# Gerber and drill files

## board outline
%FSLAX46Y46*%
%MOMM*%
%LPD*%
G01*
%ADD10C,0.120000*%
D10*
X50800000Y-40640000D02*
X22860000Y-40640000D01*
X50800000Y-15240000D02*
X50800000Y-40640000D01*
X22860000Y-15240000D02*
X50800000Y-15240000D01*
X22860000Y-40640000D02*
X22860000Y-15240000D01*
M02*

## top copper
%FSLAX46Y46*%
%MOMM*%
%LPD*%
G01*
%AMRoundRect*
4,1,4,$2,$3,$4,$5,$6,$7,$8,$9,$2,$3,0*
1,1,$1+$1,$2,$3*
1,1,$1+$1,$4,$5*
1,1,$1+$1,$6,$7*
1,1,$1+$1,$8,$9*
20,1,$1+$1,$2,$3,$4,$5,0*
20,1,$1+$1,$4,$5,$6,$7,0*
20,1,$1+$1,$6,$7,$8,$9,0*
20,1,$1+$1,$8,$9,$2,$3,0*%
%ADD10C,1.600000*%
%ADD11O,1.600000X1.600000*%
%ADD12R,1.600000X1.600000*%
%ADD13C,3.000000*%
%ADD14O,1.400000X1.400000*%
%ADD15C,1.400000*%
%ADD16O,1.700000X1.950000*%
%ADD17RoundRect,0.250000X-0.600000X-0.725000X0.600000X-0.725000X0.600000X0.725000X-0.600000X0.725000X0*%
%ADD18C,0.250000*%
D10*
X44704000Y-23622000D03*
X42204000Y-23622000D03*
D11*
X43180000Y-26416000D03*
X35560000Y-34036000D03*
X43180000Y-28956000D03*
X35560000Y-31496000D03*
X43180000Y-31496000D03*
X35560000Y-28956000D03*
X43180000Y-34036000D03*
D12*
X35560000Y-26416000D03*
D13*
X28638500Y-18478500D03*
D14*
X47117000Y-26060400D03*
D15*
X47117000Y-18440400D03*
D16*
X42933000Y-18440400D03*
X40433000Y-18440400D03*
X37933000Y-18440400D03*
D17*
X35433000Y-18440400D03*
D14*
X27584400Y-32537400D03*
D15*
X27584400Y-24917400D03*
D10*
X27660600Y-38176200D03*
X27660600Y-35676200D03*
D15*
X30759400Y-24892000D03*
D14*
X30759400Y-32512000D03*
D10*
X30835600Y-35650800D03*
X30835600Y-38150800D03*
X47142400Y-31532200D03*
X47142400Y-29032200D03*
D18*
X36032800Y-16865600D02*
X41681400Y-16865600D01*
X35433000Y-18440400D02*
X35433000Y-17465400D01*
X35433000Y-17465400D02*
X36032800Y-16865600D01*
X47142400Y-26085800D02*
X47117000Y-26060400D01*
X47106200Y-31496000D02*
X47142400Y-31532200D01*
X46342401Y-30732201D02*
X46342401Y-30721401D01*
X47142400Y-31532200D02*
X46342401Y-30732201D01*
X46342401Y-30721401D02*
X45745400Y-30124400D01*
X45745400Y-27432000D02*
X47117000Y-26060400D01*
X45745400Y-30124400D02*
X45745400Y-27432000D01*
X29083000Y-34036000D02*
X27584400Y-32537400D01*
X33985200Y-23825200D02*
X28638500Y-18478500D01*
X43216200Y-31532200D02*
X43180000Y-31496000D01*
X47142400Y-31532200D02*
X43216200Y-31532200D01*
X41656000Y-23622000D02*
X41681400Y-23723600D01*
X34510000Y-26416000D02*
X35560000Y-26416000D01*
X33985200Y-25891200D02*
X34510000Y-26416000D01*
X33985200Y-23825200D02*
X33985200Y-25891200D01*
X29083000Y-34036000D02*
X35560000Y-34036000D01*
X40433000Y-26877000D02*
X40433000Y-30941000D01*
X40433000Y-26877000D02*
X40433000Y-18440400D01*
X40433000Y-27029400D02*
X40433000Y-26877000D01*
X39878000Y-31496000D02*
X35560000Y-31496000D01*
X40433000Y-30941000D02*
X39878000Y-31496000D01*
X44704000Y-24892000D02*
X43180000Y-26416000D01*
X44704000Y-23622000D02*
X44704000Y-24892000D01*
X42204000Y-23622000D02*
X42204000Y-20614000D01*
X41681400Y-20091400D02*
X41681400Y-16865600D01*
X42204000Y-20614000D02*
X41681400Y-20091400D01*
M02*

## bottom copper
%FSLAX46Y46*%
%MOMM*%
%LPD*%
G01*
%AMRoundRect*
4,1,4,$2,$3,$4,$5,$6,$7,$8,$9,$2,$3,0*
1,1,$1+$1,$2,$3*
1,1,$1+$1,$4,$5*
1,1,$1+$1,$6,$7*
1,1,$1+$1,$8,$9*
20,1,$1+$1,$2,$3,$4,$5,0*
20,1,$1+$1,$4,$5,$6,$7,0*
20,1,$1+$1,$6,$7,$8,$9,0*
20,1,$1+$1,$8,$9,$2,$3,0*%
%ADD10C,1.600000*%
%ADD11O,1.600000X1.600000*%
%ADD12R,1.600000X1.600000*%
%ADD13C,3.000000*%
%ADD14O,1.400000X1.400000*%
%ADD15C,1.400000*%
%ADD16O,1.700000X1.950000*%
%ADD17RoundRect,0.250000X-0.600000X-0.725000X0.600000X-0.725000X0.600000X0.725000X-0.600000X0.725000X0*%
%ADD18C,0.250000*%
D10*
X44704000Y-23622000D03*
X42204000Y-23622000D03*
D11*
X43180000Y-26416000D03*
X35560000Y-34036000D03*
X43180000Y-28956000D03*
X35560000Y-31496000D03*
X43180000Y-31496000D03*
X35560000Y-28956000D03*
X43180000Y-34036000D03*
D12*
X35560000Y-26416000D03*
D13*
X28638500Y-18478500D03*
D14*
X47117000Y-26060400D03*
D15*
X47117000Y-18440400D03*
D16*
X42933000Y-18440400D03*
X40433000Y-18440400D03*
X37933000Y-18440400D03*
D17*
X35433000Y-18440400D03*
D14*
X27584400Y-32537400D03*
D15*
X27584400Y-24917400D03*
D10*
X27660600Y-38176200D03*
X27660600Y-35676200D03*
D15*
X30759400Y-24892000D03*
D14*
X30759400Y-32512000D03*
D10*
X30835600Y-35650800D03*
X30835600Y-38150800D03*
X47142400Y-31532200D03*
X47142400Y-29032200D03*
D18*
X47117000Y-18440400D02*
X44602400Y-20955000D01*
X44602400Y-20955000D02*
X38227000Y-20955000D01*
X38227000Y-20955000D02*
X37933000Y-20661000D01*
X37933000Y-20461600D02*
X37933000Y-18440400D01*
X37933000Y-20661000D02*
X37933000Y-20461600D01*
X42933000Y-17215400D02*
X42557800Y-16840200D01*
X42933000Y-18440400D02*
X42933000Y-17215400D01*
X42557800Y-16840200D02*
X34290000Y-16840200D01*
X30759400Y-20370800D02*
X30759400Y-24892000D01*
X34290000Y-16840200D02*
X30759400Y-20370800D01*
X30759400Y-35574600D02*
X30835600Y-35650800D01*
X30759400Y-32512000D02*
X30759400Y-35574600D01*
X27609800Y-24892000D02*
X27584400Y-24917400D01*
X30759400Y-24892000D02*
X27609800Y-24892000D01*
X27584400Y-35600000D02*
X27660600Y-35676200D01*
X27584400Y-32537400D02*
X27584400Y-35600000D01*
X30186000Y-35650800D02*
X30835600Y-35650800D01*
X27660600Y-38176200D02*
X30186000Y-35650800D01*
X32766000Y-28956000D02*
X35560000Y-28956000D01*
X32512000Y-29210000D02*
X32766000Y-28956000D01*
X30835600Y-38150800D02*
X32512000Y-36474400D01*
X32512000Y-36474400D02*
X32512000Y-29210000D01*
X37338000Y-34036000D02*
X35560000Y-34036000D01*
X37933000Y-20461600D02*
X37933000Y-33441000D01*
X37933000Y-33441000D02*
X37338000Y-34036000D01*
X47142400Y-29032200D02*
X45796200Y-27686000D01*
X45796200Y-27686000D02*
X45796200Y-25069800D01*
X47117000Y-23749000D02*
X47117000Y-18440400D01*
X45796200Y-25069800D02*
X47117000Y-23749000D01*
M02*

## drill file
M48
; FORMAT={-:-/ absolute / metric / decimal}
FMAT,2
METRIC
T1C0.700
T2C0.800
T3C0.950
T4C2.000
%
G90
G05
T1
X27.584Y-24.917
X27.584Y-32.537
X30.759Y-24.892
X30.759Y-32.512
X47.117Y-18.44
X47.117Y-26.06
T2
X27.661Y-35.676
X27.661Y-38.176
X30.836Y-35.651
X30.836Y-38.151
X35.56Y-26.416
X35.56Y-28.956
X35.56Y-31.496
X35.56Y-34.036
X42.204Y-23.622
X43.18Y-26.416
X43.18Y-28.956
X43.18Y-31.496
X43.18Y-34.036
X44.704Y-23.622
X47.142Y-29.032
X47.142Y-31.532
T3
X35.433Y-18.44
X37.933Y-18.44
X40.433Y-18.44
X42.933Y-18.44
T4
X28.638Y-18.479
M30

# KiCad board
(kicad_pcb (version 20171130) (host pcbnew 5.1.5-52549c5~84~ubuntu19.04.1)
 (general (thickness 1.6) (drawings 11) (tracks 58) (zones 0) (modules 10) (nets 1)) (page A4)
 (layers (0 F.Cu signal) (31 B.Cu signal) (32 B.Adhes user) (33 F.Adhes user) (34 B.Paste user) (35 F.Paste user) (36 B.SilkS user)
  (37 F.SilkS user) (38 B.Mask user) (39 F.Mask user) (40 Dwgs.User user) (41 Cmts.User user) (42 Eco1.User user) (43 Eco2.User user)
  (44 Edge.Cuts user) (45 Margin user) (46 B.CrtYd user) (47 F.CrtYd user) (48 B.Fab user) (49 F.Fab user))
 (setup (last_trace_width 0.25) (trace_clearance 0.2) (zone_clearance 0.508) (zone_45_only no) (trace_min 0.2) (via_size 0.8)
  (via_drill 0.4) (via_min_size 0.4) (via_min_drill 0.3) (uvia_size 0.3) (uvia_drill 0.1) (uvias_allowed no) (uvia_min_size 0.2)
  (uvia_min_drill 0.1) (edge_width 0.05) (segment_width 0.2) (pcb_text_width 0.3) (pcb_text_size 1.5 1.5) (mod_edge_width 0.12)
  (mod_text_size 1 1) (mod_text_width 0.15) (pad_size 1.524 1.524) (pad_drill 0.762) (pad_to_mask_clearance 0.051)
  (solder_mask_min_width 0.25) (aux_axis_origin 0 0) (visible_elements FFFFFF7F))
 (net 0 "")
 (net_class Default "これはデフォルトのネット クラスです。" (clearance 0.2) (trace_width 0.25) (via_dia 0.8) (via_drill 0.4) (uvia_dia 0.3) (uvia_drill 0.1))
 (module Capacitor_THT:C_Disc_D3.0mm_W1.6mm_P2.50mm (layer F.Cu) (at 44.704 23.622 180)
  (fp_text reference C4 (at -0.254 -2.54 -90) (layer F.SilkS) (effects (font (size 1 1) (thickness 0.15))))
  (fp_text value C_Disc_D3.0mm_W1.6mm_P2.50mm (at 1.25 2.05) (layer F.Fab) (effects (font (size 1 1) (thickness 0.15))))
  (pad 1 thru_hole circle (at 0 0 180) (size 1.6 1.6) (drill 0.8) (layers *.Cu *.Mask))
  (pad 2 thru_hole circle (at 2.5 0 180) (size 1.6 1.6) (drill 0.8) (layers *.Cu *.Mask)))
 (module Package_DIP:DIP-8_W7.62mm (layer F.Cu) (at 35.56 26.416)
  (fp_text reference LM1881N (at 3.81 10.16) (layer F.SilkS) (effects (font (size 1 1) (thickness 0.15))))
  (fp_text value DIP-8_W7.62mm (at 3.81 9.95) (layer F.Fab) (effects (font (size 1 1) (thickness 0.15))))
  (pad 8 thru_hole oval (at 7.62 0) (size 1.6 1.6) (drill 0.8) (layers *.Cu *.Mask))
  (pad 4 thru_hole oval (at 0 7.62) (size 1.6 1.6) (drill 0.8) (layers *.Cu *.Mask))
  (pad 7 thru_hole oval (at 7.62 2.54) (size 1.6 1.6) (drill 0.8) (layers *.Cu *.Mask))
  (pad 3 thru_hole oval (at 0 5.08) (size 1.6 1.6) (drill 0.8) (layers *.Cu *.Mask))
  (pad 6 thru_hole oval (at 7.62 5.08) (size 1.6 1.6) (drill 0.8) (layers *.Cu *.Mask))
  (pad 2 thru_hole oval (at 0 2.54) (size 1.6 1.6) (drill 0.8) (layers *.Cu *.Mask))
  (pad 5 thru_hole oval (at 7.62 7.62) (size 1.6 1.6) (drill 0.8) (layers *.Cu *.Mask))
  (pad 1 thru_hole rect (at 0 0) (size 1.6 1.6) (drill 0.8) (layers *.Cu *.Mask)))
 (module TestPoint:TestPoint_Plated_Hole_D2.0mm (layer F.Cu) (at 28.6385 18.4785)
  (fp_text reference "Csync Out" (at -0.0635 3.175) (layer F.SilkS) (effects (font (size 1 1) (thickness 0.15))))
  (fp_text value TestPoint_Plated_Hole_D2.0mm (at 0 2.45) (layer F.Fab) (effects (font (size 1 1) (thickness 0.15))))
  (pad 1 thru_hole circle (at 0 0) (size 3 3) (drill 2) (layers *.Cu *.Mask)))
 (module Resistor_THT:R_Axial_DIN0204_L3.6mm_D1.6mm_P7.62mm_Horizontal (layer F.Cu) (at 47.117 18.4404 270)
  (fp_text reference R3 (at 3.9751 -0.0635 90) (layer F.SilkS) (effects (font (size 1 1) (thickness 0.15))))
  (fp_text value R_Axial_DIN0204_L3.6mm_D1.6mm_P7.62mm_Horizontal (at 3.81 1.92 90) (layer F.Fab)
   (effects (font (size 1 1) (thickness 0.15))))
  (pad 2 thru_hole oval (at 7.62 0 270) (size 1.4 1.4) (drill 0.7) (layers *.Cu *.Mask))
  (pad 1 thru_hole circle (at 0 0 270) (size 1.4 1.4) (drill 0.7) (layers *.Cu *.Mask)))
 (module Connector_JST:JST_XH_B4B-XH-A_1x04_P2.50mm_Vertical (layer F.Cu) (at 35.433 18.4404)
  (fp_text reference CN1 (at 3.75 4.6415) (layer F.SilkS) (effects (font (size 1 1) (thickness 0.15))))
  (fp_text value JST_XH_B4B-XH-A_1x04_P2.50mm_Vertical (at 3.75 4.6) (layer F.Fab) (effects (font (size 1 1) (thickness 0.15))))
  (pad 4 thru_hole oval (at 7.5 0) (size 1.7 1.95) (drill 0.95) (layers *.Cu *.Mask))
  (pad 3 thru_hole oval (at 5 0) (size 1.7 1.95) (drill 0.95) (layers *.Cu *.Mask))
  (pad 2 thru_hole oval (at 2.5 0) (size 1.7 1.95) (drill 0.95) (layers *.Cu *.Mask))
  (pad 1 thru_hole roundrect (at 0 0) (size 1.7 1.95) (drill 0.95) (layers *.Cu *.Mask) (roundrect_rratio 0.147059)))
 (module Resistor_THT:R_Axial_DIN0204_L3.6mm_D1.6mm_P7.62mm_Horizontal (layer F.Cu) (at 27.5844 24.9174 270)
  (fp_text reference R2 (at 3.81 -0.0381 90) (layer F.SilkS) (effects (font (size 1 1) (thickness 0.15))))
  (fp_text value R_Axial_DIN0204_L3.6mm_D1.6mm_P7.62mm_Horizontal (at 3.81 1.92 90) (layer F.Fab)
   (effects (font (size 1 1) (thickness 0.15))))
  (pad 2 thru_hole oval (at 7.62 0 270) (size 1.4 1.4) (drill 0.7) (layers *.Cu *.Mask))
  (pad 1 thru_hole circle (at 0 0 270) (size 1.4 1.4) (drill 0.7) (layers *.Cu *.Mask)))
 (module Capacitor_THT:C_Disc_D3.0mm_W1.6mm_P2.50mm (layer F.Cu) (at 27.6606 35.6762 270)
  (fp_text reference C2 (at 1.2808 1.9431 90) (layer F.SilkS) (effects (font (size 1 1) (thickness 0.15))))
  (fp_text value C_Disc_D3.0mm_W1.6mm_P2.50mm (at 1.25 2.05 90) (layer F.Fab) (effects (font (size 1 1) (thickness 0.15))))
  (pad 2 thru_hole circle (at 2.5 0 270) (size 1.6 1.6) (drill 0.8) (layers *.Cu *.Mask))
  (pad 1 thru_hole circle (at 0 0 270) (size 1.6 1.6) (drill 0.8) (layers *.Cu *.Mask)))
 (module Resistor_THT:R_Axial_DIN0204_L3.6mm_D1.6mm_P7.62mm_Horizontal (layer F.Cu) (at 30.7594 24.892 270)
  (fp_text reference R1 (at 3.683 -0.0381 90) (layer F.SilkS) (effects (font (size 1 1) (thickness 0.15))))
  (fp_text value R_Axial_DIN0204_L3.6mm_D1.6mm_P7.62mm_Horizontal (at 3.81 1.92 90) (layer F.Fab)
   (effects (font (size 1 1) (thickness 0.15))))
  (pad 1 thru_hole circle (at 0 0 270) (size 1.4 1.4) (drill 0.7) (layers *.Cu *.Mask))
  (pad 2 thru_hole oval (at 7.62 0 270) (size 1.4 1.4) (drill 0.7) (layers *.Cu *.Mask)))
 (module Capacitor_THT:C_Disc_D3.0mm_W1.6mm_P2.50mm (layer F.Cu) (at 30.8356 35.6508 270)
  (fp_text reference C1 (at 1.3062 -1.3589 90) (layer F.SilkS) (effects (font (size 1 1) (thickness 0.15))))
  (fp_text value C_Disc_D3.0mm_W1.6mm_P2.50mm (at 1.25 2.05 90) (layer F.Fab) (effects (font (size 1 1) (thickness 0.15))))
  (pad 1 thru_hole circle (at 0 0 270) (size 1.6 1.6) (drill 0.8) (layers *.Cu *.Mask))
  (pad 2 thru_hole circle (at 2.5 0 270) (size 1.6 1.6) (drill 0.8) (layers *.Cu *.Mask)))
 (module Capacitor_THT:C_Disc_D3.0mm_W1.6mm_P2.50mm (layer F.Cu) (at 47.1424 29.0322 270)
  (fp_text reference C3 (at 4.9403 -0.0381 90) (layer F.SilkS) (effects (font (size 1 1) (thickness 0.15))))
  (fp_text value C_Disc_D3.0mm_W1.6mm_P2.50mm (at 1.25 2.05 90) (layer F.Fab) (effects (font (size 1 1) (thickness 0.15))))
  (pad 2 thru_hole circle (at 2.5 0 270) (size 1.6 1.6) (drill 0.8) (layers *.Cu *.Mask))
  (pad 1 thru_hole circle (at 0 0 270) (size 1.6 1.6) (drill 0.8) (layers *.Cu *.Mask)))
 (gr_line (start 50.8 40.64) (end 22.86 40.64) (layer Edge.Cuts) (width 0.12))
 (gr_line (start 50.8 15.24) (end 50.8 40.64) (layer Edge.Cuts) (width 0.12))
 (gr_line (start 22.86 15.24) (end 50.8 15.24) (layer Edge.Cuts) (width 0.12))
 (gr_line (start 22.86 40.64) (end 22.86 15.24) (layer Edge.Cuts) (width 0.12))
 (segment (start 36.0328 16.8656) (end 41.6814 16.8656) (width 0.25) (layer F.Cu) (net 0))
 (segment (start 35.433 18.4404) (end 35.433 17.4654) (width 0.25) (layer F.Cu) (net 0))
 (segment (start 35.433 17.4654) (end 36.0328 16.8656) (width 0.25) (layer F.Cu) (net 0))
 (segment (start 47.1424 26.0858) (end 47.117 26.0604) (width 0.25) (layer F.Cu) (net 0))
 (segment (start 47.1062 31.496) (end 47.1424 31.5322) (width 0.25) (layer F.Cu) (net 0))
 (segment (start 46.342401 30.732201) (end 46.342401 30.721401) (width 0.25) (layer F.Cu) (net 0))
 (segment (start 47.1424 31.5322) (end 46.342401 30.732201) (width 0.25) (layer F.Cu) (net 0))
 (segment (start 46.342401 30.721401) (end 45.7454 30.1244) (width 0.25) (layer F.Cu) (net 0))
 (segment (start 45.7454 27.432) (end 47.117 26.0604) (width 0.25) (layer F.Cu) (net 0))
 (segment (start 45.7454 30.1244) (end 45.7454 27.432) (width 0.25) (layer F.Cu) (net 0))
 (segment (start 47.117 18.4404) (end 44.6024 20.955) (width 0.25) (layer B.Cu) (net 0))
 (segment (start 44.6024 20.955) (end 38.227 20.955) (width 0.25) (layer B.Cu) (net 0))
 (segment (start 38.227 20.955) (end 37.933 20.661) (width 0.25) (layer B.Cu) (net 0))
 (segment (start 37.933 20.4616) (end 37.933 18.4404) (width 0.25) (layer B.Cu) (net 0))
 (segment (start 37.933 20.661) (end 37.933 20.4616) (width 0.25) (layer B.Cu) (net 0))
 (segment (start 42.933 17.2154) (end 42.5578 16.8402) (width 0.25) (layer B.Cu) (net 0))
 (segment (start 42.933 18.4404) (end 42.933 17.2154) (width 0.25) (layer B.Cu) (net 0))
 (segment (start 42.5578 16.8402) (end 34.29 16.8402) (width 0.25) (layer B.Cu) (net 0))
 (segment (start 30.7594 20.3708) (end 30.7594 24.892) (width 0.25) (layer B.Cu) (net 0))
 (segment (start 34.29 16.8402) (end 30.7594 20.3708) (width 0.25) (layer B.Cu) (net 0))
 (segment (start 30.7594 35.5746) (end 30.8356 35.6508) (width 0.25) (layer B.Cu) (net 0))
 (segment (start 30.7594 32.512) (end 30.7594 35.5746) (width 0.25) (layer B.Cu) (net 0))
 (segment (start 27.6098 24.892) (end 27.5844 24.9174) (width 0.25) (layer B.Cu) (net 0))
 (segment (start 30.7594 24.892) (end 27.6098 24.892) (width 0.25) (layer B.Cu) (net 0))
 (segment (start 27.5844 35.6) (end 27.6606 35.6762) (width 0.25) (layer B.Cu) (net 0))
 (segment (start 27.5844 32.5374) (end 27.5844 35.6) (width 0.25) (layer B.Cu) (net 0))
 (segment (start 29.083 34.036) (end 27.5844 32.5374) (width 0.25) (layer F.Cu) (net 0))
 (segment (start 30.186 35.6508) (end 30.8356 35.6508) (width 0.25) (layer B.Cu) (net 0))
 (segment (start 27.6606 38.1762) (end 30.186 35.6508) (width 0.25) (layer B.Cu) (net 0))
 (segment (start 33.9852 23.8252) (end 28.6385 18.4785) (width 0.25) (layer F.Cu) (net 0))
 (segment (start 43.2162 31.5322) (end 43.18 31.496) (width 0.25) (layer F.Cu) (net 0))
 (segment (start 47.1424 31.5322) (end 43.2162 31.5322) (width 0.25) (layer F.Cu) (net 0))
 (segment (start 41.656 23.622) (end 41.6814 23.7236) (width 0.25) (layer F.Cu) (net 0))
 (segment (start 34.51 26.416) (end 35.56 26.416) (width 0.25) (layer F.Cu) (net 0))
 (segment (start 33.9852 25.8912) (end 34.51 26.416) (width 0.25) (layer F.Cu) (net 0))
 (segment (start 33.9852 23.8252) (end 33.9852 25.8912) (width 0.25) (layer F.Cu) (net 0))
 (segment (start 29.083 34.036) (end 35.56 34.036) (width 0.25) (layer F.Cu) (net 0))
 (segment (start 32.766 28.956) (end 35.56 28.956) (width 0.25) (layer B.Cu) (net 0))
 (segment (start 32.512 29.21) (end 32.766 28.956) (width 0.25) (layer B.Cu) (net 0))
 (segment (start 30.8356 38.1508) (end 32.512 36.4744) (width 0.25) (layer B.Cu) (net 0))
 (segment (start 32.512 36.4744) (end 32.512 29.21) (width 0.25) (layer B.Cu) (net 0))
 (segment (start 37.338 34.036) (end 35.56 34.036) (width 0.25) (layer B.Cu) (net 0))
 (segment (start 37.933 20.4616) (end 37.933 33.441) (width 0.25) (layer B.Cu) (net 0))
 (segment (start 37.933 33.441) (end 37.338 34.036) (width 0.25) (layer B.Cu) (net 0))
 (segment (start 40.433 26.877) (end 40.433 30.941) (width 0.25) (layer F.Cu) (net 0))
 (segment (start 40.433 26.877) (end 40.433 18.4404) (width 0.25) (layer F.Cu) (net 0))
 (segment (start 40.433 27.0294) (end 40.433 26.877) (width 0.25) (layer F.Cu) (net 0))
 (segment (start 39.878 31.496) (end 35.56 31.496) (width 0.25) (layer F.Cu) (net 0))
 (segment (start 40.433 30.941) (end 39.878 31.496) (width 0.25) (layer F.Cu) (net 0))
 (segment (start 44.704 24.892) (end 43.18 26.416) (width 0.25) (layer F.Cu) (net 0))
 (segment (start 44.704 23.622) (end 44.704 24.892) (width 0.25) (layer F.Cu) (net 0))
 (segment (start 42.204 23.622) (end 42.204 20.614) (width 0.25) (layer F.Cu) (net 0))
 (segment (start 41.6814 20.0914) (end 41.6814 16.8656) (width 0.25) (layer F.Cu) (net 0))
 (segment (start 42.204 20.614) (end 41.6814 20.0914) (width 0.25) (layer F.Cu) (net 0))
 (segment (start 47.1424 29.0322) (end 45.7962 27.686) (width 0.25) (layer B.Cu) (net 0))
 (segment (start 45.7962 27.686) (end 45.7962 25.0698) (width 0.25) (layer B.Cu) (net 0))
 (segment (start 47.117 23.749) (end 47.117 18.4404) (width 0.25) (layer B.Cu) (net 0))
 (segment (start 45.7962 25.0698) (end 47.117 23.749) (width 0.25) (layer B.Cu) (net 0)))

